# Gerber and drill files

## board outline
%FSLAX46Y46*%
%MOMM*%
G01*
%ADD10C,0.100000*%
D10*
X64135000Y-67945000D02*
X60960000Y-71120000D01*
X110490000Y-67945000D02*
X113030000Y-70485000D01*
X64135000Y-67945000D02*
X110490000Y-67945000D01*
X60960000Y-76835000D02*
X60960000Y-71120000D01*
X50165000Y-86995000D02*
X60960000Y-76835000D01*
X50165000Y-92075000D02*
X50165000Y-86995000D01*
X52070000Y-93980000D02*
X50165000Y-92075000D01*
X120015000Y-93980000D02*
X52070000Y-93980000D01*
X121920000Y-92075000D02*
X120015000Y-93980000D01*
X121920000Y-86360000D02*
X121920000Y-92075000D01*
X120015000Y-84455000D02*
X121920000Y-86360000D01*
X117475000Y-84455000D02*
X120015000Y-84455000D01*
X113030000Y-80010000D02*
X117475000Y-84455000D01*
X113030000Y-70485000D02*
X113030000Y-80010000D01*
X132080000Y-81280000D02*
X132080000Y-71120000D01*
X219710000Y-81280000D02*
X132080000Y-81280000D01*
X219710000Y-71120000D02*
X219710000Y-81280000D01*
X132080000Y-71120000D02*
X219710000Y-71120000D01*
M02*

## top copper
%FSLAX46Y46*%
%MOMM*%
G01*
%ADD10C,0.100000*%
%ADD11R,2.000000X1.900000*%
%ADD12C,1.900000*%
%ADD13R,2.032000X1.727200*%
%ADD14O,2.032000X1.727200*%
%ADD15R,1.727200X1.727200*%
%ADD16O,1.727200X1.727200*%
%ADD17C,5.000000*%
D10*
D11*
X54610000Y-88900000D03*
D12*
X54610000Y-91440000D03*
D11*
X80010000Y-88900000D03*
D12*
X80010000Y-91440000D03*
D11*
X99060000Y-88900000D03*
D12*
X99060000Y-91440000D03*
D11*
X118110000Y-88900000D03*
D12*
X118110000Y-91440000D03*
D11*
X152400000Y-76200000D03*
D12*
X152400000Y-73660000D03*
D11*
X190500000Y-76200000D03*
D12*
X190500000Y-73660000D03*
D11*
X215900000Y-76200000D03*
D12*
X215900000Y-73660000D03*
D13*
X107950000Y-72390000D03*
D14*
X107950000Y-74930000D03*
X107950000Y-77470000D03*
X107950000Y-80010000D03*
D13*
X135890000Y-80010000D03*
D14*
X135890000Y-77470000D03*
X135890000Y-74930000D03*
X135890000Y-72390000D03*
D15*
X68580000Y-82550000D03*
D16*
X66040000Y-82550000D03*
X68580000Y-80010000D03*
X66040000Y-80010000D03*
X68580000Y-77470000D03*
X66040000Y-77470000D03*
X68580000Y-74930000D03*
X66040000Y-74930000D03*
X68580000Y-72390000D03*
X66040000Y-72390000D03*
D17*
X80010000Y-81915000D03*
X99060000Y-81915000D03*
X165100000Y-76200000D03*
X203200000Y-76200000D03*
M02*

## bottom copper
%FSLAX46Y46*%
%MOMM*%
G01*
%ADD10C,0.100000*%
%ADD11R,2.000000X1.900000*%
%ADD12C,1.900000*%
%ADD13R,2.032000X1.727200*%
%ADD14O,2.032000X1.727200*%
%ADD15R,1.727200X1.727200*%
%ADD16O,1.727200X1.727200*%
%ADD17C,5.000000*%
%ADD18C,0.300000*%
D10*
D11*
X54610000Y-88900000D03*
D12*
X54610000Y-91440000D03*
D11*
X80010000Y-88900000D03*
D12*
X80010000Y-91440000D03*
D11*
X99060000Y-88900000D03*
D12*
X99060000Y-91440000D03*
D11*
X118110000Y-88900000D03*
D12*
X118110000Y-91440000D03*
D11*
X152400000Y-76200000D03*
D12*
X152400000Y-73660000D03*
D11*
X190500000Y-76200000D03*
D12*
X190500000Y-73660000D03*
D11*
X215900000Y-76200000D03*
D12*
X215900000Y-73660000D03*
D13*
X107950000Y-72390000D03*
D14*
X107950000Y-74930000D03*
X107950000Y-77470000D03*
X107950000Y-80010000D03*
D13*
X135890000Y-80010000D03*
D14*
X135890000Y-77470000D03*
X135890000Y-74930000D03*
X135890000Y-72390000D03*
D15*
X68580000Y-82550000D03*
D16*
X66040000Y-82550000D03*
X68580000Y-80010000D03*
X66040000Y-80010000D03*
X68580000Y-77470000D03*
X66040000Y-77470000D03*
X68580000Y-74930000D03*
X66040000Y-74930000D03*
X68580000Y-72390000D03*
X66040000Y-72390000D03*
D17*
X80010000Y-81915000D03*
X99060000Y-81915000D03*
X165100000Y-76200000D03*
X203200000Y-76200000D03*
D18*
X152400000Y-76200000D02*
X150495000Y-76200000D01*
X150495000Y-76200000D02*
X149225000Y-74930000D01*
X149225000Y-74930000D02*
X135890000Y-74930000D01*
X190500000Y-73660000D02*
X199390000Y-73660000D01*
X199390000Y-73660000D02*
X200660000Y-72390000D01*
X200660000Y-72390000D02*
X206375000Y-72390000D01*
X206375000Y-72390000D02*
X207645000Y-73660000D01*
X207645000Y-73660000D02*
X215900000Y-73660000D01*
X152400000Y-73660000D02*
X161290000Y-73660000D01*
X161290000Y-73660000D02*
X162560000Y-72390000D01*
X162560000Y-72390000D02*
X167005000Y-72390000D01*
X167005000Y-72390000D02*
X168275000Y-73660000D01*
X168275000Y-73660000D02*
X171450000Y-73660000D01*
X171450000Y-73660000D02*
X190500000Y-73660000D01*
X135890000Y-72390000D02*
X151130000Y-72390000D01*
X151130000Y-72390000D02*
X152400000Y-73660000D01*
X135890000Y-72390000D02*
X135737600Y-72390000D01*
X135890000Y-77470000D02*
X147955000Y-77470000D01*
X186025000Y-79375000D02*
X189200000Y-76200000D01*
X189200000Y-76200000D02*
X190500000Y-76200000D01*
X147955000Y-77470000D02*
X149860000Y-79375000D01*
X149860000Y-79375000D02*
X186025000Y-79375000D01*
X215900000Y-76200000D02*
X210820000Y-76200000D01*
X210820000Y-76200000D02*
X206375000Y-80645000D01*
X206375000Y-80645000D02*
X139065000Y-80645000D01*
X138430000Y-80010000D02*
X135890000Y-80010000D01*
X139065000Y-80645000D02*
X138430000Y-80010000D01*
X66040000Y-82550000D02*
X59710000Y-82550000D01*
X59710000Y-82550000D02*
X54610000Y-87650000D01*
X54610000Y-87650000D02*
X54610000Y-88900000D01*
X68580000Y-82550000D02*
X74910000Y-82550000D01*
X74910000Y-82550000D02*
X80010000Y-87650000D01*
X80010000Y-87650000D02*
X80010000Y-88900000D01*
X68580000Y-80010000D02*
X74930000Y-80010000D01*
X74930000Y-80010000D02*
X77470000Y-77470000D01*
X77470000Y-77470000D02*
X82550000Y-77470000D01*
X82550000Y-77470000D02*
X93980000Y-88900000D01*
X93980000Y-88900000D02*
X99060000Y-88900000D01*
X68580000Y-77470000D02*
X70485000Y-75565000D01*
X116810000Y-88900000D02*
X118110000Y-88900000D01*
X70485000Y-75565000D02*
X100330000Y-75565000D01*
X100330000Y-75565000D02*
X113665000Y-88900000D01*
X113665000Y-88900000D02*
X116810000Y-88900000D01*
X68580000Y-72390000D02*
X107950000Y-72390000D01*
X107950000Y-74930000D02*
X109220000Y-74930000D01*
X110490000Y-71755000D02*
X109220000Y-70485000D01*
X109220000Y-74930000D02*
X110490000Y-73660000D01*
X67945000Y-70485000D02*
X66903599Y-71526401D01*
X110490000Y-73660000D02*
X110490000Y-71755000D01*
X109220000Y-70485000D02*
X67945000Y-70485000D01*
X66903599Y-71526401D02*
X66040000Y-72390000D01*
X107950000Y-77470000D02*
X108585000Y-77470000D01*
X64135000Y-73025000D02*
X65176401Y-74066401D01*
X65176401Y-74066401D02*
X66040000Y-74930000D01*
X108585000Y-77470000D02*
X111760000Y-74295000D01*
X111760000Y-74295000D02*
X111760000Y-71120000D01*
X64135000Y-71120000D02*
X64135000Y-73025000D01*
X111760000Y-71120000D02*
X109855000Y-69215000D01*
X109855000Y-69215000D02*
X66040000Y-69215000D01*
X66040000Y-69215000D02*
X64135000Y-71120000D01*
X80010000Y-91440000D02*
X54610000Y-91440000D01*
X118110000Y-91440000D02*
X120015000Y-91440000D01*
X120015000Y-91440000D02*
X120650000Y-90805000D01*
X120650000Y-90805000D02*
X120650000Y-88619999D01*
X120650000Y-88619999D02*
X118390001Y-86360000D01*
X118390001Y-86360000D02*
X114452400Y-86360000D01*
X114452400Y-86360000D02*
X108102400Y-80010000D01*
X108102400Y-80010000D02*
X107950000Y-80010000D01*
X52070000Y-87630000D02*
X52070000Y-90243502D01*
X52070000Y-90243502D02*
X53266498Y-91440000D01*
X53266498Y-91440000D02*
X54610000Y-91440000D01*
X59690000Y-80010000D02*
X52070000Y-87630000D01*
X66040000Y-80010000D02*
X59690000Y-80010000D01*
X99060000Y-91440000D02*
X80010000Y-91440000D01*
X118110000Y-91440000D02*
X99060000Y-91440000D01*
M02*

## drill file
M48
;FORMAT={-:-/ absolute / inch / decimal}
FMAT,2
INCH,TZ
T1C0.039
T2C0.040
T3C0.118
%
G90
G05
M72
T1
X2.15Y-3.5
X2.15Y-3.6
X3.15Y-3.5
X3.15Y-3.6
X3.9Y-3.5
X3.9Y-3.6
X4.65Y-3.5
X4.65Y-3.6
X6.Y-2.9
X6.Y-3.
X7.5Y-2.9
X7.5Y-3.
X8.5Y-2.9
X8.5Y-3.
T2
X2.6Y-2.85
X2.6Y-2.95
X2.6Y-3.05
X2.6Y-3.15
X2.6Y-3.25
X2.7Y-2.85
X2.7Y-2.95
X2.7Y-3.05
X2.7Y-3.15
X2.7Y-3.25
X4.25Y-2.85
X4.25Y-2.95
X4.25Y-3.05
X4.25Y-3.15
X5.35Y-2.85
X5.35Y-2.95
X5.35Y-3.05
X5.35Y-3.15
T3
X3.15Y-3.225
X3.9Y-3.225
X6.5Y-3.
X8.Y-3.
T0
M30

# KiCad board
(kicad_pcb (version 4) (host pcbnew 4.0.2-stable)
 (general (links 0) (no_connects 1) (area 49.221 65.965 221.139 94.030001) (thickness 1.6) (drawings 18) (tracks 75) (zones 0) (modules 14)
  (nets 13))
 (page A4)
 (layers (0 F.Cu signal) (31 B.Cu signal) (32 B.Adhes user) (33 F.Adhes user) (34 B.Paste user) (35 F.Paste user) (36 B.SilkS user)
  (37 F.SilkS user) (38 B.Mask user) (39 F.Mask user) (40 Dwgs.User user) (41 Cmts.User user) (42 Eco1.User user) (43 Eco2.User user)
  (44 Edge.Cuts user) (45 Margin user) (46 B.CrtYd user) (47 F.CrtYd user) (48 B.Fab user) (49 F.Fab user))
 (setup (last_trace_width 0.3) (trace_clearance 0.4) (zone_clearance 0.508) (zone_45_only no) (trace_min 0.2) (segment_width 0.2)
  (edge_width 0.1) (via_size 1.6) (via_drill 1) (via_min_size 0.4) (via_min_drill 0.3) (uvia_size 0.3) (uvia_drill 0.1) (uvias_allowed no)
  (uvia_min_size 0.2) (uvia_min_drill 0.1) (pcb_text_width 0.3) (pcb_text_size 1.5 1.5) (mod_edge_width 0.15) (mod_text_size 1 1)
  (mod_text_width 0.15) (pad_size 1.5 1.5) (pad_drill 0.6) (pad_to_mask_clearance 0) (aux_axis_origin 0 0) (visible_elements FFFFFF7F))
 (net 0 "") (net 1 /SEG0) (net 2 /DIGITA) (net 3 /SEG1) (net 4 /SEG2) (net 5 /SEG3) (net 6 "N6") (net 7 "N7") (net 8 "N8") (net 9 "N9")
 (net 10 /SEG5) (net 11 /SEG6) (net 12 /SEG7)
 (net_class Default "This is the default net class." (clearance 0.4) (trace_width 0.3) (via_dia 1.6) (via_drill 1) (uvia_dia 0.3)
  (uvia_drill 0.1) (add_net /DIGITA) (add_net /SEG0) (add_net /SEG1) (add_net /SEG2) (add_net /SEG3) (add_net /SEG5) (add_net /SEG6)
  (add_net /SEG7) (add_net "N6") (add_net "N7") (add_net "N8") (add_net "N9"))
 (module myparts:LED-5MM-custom (layer F.Cu) (at 54.61 88.9 270)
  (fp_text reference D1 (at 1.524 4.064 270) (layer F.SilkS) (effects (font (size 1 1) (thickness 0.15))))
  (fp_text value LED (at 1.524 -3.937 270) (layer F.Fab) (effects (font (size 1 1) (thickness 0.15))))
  (pad 1 thru_hole rect (at 0 0) (size 2 1.9) (drill 1.00076) (layers *.Cu *.Mask F.SilkS) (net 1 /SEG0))
  (pad 2 thru_hole circle (at 2.54 0 270) (size 1.9 1.9) (drill 1.00076) (layers *.Cu *.Mask F.SilkS) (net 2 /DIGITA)))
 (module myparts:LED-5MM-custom (layer F.Cu) (at 80.01 88.9 270)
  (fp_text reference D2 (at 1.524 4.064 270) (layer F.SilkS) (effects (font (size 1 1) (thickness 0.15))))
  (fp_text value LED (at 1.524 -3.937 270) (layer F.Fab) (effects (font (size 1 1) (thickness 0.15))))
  (pad 1 thru_hole rect (at 0 0) (size 2 1.9) (drill 1.00076) (layers *.Cu *.Mask F.SilkS) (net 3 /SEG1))
  (pad 2 thru_hole circle (at 2.54 0 270) (size 1.9 1.9) (drill 1.00076) (layers *.Cu *.Mask F.SilkS) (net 2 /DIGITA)))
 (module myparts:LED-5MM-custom (layer F.Cu) (at 99.06 88.9 270)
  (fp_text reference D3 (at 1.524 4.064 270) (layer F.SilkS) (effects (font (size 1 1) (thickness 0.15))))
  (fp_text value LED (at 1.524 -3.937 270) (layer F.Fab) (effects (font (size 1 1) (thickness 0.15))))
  (pad 1 thru_hole rect (at 0 0) (size 2 1.9) (drill 1.00076) (layers *.Cu *.Mask F.SilkS) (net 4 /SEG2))
  (pad 2 thru_hole circle (at 2.54 0 270) (size 1.9 1.9) (drill 1.00076) (layers *.Cu *.Mask F.SilkS) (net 2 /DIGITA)))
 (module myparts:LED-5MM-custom (layer F.Cu) (at 118.11 88.9 270)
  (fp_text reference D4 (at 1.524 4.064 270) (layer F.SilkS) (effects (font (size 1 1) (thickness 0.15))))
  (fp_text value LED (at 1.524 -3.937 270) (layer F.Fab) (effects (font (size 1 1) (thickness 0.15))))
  (pad 1 thru_hole rect (at 0 0) (size 2 1.9) (drill 1.00076) (layers *.Cu *.Mask F.SilkS) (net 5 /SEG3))
  (pad 2 thru_hole circle (at 2.54 0 270) (size 1.9 1.9) (drill 1.00076) (layers *.Cu *.Mask F.SilkS) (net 2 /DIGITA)))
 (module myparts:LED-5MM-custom (layer F.Cu) (at 152.4 76.2 90)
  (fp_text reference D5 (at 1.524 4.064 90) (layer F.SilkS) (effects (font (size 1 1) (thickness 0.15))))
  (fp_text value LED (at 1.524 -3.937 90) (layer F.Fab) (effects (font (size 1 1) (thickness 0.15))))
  (pad 1 thru_hole rect (at 0 0 180) (size 2 1.9) (drill 1.00076) (layers *.Cu *.Mask F.SilkS) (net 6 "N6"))
  (pad 2 thru_hole circle (at 2.54 0 90) (size 1.9 1.9) (drill 1.00076) (layers *.Cu *.Mask F.SilkS) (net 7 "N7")))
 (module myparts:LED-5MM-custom (layer F.Cu) (at 190.5 76.2 90)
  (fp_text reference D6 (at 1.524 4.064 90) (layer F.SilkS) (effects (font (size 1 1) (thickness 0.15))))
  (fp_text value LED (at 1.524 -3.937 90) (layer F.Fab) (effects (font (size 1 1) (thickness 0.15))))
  (pad 1 thru_hole rect (at 0 0 180) (size 2 1.9) (drill 1.00076) (layers *.Cu *.Mask F.SilkS) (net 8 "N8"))
  (pad 2 thru_hole circle (at 2.54 0 90) (size 1.9 1.9) (drill 1.00076) (layers *.Cu *.Mask F.SilkS) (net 7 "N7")))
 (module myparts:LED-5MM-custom (layer F.Cu) (at 215.9 76.2 90)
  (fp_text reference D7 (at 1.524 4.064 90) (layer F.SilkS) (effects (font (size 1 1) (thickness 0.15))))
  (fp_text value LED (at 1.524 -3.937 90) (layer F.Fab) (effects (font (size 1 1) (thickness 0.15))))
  (pad 1 thru_hole rect (at 0 0 180) (size 2 1.9) (drill 1.00076) (layers *.Cu *.Mask F.SilkS) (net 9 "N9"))
  (pad 2 thru_hole circle (at 2.54 0 90) (size 1.9 1.9) (drill 1.00076) (layers *.Cu *.Mask F.SilkS) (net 7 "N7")))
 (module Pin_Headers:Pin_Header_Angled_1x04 (layer F.Cu) (at 107.95 72.39)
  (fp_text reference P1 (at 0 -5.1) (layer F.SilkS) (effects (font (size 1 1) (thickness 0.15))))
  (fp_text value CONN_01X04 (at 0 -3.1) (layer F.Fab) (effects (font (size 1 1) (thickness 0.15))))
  (pad 1 thru_hole rect (at 0 0) (size 2.032 1.7272) (drill 1.016) (layers *.Cu *.Mask F.SilkS) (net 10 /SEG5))
  (pad 2 thru_hole oval (at 0 2.54) (size 2.032 1.7272) (drill 1.016) (layers *.Cu *.Mask F.SilkS) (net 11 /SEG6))
  (pad 3 thru_hole oval (at 0 5.08) (size 2.032 1.7272) (drill 1.016) (layers *.Cu *.Mask F.SilkS) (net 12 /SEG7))
  (pad 4 thru_hole oval (at 0 7.62) (size 2.032 1.7272) (drill 1.016) (layers *.Cu *.Mask F.SilkS) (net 2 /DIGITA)))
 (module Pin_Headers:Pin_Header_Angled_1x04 (layer F.Cu) (at 135.89 80.01 180)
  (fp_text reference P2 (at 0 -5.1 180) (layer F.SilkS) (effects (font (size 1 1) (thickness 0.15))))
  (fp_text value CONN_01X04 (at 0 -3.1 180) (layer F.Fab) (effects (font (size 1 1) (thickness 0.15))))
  (pad 1 thru_hole rect (at 0 0 180) (size 2.032 1.7272) (drill 1.016) (layers *.Cu *.Mask F.SilkS) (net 9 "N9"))
  (pad 2 thru_hole oval (at 0 2.54 180) (size 2.032 1.7272) (drill 1.016) (layers *.Cu *.Mask F.SilkS) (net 8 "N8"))
  (pad 3 thru_hole oval (at 0 5.08 180) (size 2.032 1.7272) (drill 1.016) (layers *.Cu *.Mask F.SilkS) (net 6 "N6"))
  (pad 4 thru_hole oval (at 0 7.62 180) (size 2.032 1.7272) (drill 1.016) (layers *.Cu *.Mask F.SilkS) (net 7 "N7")))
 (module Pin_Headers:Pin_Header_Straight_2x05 (layer F.Cu) (at 68.58 82.55 180)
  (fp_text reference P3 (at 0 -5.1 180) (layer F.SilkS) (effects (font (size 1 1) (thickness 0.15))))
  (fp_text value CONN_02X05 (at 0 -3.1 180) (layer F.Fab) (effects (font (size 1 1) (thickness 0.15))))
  (pad 1 thru_hole rect (at 0 0 180) (size 1.7272 1.7272) (drill 1.016) (layers *.Cu *.Mask F.SilkS) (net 3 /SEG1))
  (pad 2 thru_hole oval (at 2.54 0 180) (size 1.7272 1.7272) (drill 1.016) (layers *.Cu *.Mask F.SilkS) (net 1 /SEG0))
  (pad 3 thru_hole oval (at 0 2.54 180) (size 1.7272 1.7272) (drill 1.016) (layers *.Cu *.Mask F.SilkS) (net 4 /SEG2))
  (pad 4 thru_hole oval (at 2.54 2.54 180) (size 1.7272 1.7272) (drill 1.016) (layers *.Cu *.Mask F.SilkS) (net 2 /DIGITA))
  (pad 5 thru_hole oval (at 0 5.08 180) (size 1.7272 1.7272) (drill 1.016) (layers *.Cu *.Mask F.SilkS) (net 5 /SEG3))
  (pad 6 thru_hole oval (at 2.54 5.08 180) (size 1.7272 1.7272) (drill 1.016) (layers *.Cu *.Mask F.SilkS))
  (pad 7 thru_hole oval (at 0 7.62 180) (size 1.7272 1.7272) (drill 1.016) (layers *.Cu *.Mask F.SilkS))
  (pad 8 thru_hole oval (at 2.54 7.62 180) (size 1.7272 1.7272) (drill 1.016) (layers *.Cu *.Mask F.SilkS) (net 12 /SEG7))
  (pad 9 thru_hole oval (at 0 10.16 180) (size 1.7272 1.7272) (drill 1.016) (layers *.Cu *.Mask F.SilkS) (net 10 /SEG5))
  (pad 10 thru_hole oval (at 2.54 10.16 180) (size 1.7272 1.7272) (drill 1.016) (layers *.Cu *.Mask F.SilkS) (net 11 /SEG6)))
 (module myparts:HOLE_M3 (layer F.Cu) (at 80.01 81.915)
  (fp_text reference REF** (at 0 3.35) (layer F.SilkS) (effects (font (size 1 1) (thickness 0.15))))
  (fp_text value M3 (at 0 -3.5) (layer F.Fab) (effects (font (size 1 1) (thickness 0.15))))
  (pad 1 thru_hole circle (at 0 0) (size 5 5) (drill 3) (layers *.Cu *.Mask F.SilkS)))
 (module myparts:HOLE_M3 (layer F.Cu) (at 99.06 81.915)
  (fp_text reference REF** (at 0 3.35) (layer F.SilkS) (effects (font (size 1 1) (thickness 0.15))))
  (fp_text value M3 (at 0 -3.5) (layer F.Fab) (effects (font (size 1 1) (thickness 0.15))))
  (pad 1 thru_hole circle (at 0 0) (size 5 5) (drill 3) (layers *.Cu *.Mask F.SilkS)))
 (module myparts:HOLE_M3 (layer F.Cu) (at 165.1 76.2)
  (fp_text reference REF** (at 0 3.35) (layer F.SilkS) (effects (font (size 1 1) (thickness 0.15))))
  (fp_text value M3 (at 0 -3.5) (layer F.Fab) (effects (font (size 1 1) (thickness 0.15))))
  (pad 1 thru_hole circle (at 0 0) (size 5 5) (drill 3) (layers *.Cu *.Mask F.SilkS)))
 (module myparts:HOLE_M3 (layer F.Cu) (at 203.2 76.2)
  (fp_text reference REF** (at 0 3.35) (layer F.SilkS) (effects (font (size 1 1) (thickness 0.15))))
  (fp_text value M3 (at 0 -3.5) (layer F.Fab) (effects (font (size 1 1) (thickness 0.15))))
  (pad 1 thru_hole circle (at 0 0) (size 5 5) (drill 3) (layers *.Cu *.Mask F.SilkS)))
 (gr_line (start 64.135 67.945) (end 60.96 71.12) (layer Edge.Cuts) (width 0.1))
 (gr_line (start 110.49 67.945) (end 113.03 70.485) (layer Edge.Cuts) (width 0.1))
 (gr_line (start 64.135 67.945) (end 110.49 67.945) (layer Edge.Cuts) (width 0.1))
 (gr_line (start 60.96 76.835) (end 60.96 71.12) (layer Edge.Cuts) (width 0.1))
 (gr_line (start 50.165 86.995) (end 60.96 76.835) (layer Edge.Cuts) (width 0.1))
 (gr_line (start 50.165 92.075) (end 50.165 86.995) (layer Edge.Cuts) (width 0.1))
 (gr_line (start 52.07 93.98) (end 50.165 92.075) (layer Edge.Cuts) (width 0.1))
 (gr_line (start 120.015 93.98) (end 52.07 93.98) (layer Edge.Cuts) (width 0.1))
 (gr_line (start 121.92 92.075) (end 120.015 93.98) (layer Edge.Cuts) (width 0.1))
 (gr_line (start 121.92 86.36) (end 121.92 92.075) (layer Edge.Cuts) (width 0.1))
 (gr_line (start 120.015 84.455) (end 121.92 86.36) (layer Edge.Cuts) (width 0.1))
 (gr_line (start 117.475 84.455) (end 120.015 84.455) (layer Edge.Cuts) (width 0.1))
 (gr_line (start 113.03 80.01) (end 117.475 84.455) (layer Edge.Cuts) (width 0.1))
 (gr_line (start 113.03 70.485) (end 113.03 80.01) (layer Edge.Cuts) (width 0.1))
 (gr_line (start 132.08 81.28) (end 132.08 71.12) (layer Edge.Cuts) (width 0.1))
 (gr_line (start 219.71 81.28) (end 132.08 81.28) (layer Edge.Cuts) (width 0.1))
 (gr_line (start 219.71 71.12) (end 219.71 81.28) (layer Edge.Cuts) (width 0.1))
 (gr_line (start 132.08 71.12) (end 219.71 71.12) (layer Edge.Cuts) (width 0.1))
 (segment (start 152.4 76.2) (end 150.495 76.2) (width 0.3) (layer B.Cu) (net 6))
 (segment (start 150.495 76.2) (end 149.225 74.93) (width 0.3) (layer B.Cu) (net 6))
 (segment (start 149.225 74.93) (end 135.89 74.93) (width 0.3) (layer B.Cu) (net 6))
 (segment (start 190.5 73.66) (end 199.39 73.66) (width 0.3) (layer B.Cu) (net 7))
 (segment (start 199.39 73.66) (end 200.66 72.39) (width 0.3) (layer B.Cu) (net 7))
 (segment (start 200.66 72.39) (end 206.375 72.39) (width 0.3) (layer B.Cu) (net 7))
 (segment (start 206.375 72.39) (end 207.645 73.66) (width 0.3) (layer B.Cu) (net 7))
 (segment (start 207.645 73.66) (end 215.9 73.66) (width 0.3) (layer B.Cu) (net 7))
 (segment (start 152.4 73.66) (end 161.29 73.66) (width 0.3) (layer B.Cu) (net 7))
 (segment (start 161.29 73.66) (end 162.56 72.39) (width 0.3) (layer B.Cu) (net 7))
 (segment (start 162.56 72.39) (end 167.005 72.39) (width 0.3) (layer B.Cu) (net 7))
 (segment (start 167.005 72.39) (end 168.275 73.66) (width 0.3) (layer B.Cu) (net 7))
 (segment (start 168.275 73.66) (end 171.45 73.66) (width 0.3) (layer B.Cu) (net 7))
 (segment (start 171.45 73.66) (end 190.5 73.66) (width 0.3) (layer B.Cu) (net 7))
 (segment (start 135.89 72.39) (end 151.13 72.39) (width 0.3) (layer B.Cu) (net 7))
 (segment (start 151.13 72.39) (end 152.4 73.66) (width 0.3) (layer B.Cu) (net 7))
 (segment (start 135.89 72.39) (end 135.7376 72.39) (width 0.3) (layer B.Cu) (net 7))
 (segment (start 135.89 77.47) (end 147.955 77.47) (width 0.3) (layer B.Cu) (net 8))
 (segment (start 186.025 79.375) (end 189.2 76.2) (width 0.3) (layer B.Cu) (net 8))
 (segment (start 189.2 76.2) (end 190.5 76.2) (width 0.3) (layer B.Cu) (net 8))
 (segment (start 147.955 77.47) (end 149.86 79.375) (width 0.3) (layer B.Cu) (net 8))
 (segment (start 149.86 79.375) (end 186.025 79.375) (width 0.3) (layer B.Cu) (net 8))
 (segment (start 215.9 76.2) (end 210.82 76.2) (width 0.3) (layer B.Cu) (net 9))
 (segment (start 210.82 76.2) (end 206.375 80.645) (width 0.3) (layer B.Cu) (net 9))
 (segment (start 206.375 80.645) (end 139.065 80.645) (width 0.3) (layer B.Cu) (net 9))
 (segment (start 138.43 80.01) (end 135.89 80.01) (width 0.3) (layer B.Cu) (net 9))
 (segment (start 139.065 80.645) (end 138.43 80.01) (width 0.3) (layer B.Cu) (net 9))
 (segment (start 66.04 82.55) (end 59.71 82.55) (width 0.3) (layer B.Cu) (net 1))
 (segment (start 59.71 82.55) (end 54.61 87.65) (width 0.3) (layer B.Cu) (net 1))
 (segment (start 54.61 87.65) (end 54.61 88.9) (width 0.3) (layer B.Cu) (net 1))
 (segment (start 68.58 82.55) (end 74.91 82.55) (width 0.3) (layer B.Cu) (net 3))
 (segment (start 74.91 82.55) (end 80.01 87.65) (width 0.3) (layer B.Cu) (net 3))
 (segment (start 80.01 87.65) (end 80.01 88.9) (width 0.3) (layer B.Cu) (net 3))
 (segment (start 68.58 80.01) (end 74.93 80.01) (width 0.3) (layer B.Cu) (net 4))
 (segment (start 74.93 80.01) (end 77.47 77.47) (width 0.3) (layer B.Cu) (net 4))
 (segment (start 77.47 77.47) (end 82.55 77.47) (width 0.3) (layer B.Cu) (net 4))
 (segment (start 82.55 77.47) (end 93.98 88.9) (width 0.3) (layer B.Cu) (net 4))
 (segment (start 93.98 88.9) (end 99.06 88.9) (width 0.3) (layer B.Cu) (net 4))
 (segment (start 68.58 77.47) (end 70.485 75.565) (width 0.3) (layer B.Cu) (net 5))
 (segment (start 116.81 88.9) (end 118.11 88.9) (width 0.3) (layer B.Cu) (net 5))
 (segment (start 70.485 75.565) (end 100.33 75.565) (width 0.3) (layer B.Cu) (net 5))
 (segment (start 100.33 75.565) (end 113.665 88.9) (width 0.3) (layer B.Cu) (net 5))
 (segment (start 113.665 88.9) (end 116.81 88.9) (width 0.3) (layer B.Cu) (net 5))
 (segment (start 68.58 72.39) (end 107.95 72.39) (width 0.3) (layer B.Cu) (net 10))
 (segment (start 107.95 74.93) (end 109.22 74.93) (width 0.3) (layer B.Cu) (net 11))
 (segment (start 110.49 71.755) (end 109.22 70.485) (width 0.3) (layer B.Cu) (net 11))
 (segment (start 109.22 74.93) (end 110.49 73.66) (width 0.3) (layer B.Cu) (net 11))
 (segment (start 67.945 70.485) (end 66.903599 71.526401) (width 0.3) (layer B.Cu) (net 11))
 (segment (start 110.49 73.66) (end 110.49 71.755) (width 0.3) (layer B.Cu) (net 11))
 (segment (start 109.22 70.485) (end 67.945 70.485) (width 0.3) (layer B.Cu) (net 11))
 (segment (start 66.903599 71.526401) (end 66.04 72.39) (width 0.3) (layer B.Cu) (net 11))
 (segment (start 107.95 77.47) (end 108.585 77.47) (width 0.3) (layer B.Cu) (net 12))
 (segment (start 64.135 73.025) (end 65.176401 74.066401) (width 0.3) (layer B.Cu) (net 12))
 (segment (start 65.176401 74.066401) (end 66.04 74.93) (width 0.3) (layer B.Cu) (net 12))
 (segment (start 108.585 77.47) (end 111.76 74.295) (width 0.3) (layer B.Cu) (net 12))
 (segment (start 111.76 74.295) (end 111.76 71.12) (width 0.3) (layer B.Cu) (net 12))
 (segment (start 64.135 71.12) (end 64.135 73.025) (width 0.3) (layer B.Cu) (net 12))
 (segment (start 111.76 71.12) (end 109.855 69.215) (width 0.3) (layer B.Cu) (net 12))
 (segment (start 109.855 69.215) (end 66.04 69.215) (width 0.3) (layer B.Cu) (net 12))
 (segment (start 66.04 69.215) (end 64.135 71.12) (width 0.3) (layer B.Cu) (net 12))
 (segment (start 80.01 91.44) (end 54.61 91.44) (width 0.3) (layer B.Cu) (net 2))
 (segment (start 118.11 91.44) (end 120.015 91.44) (width 0.3) (layer B.Cu) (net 2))
 (segment (start 120.015 91.44) (end 120.65 90.805) (width 0.3) (layer B.Cu) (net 2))
 (segment (start 120.65 90.805) (end 120.65 88.619999) (width 0.3) (layer B.Cu) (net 2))
 (segment (start 120.65 88.619999) (end 118.390001 86.36) (width 0.3) (layer B.Cu) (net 2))
 (segment (start 118.390001 86.36) (end 114.4524 86.36) (width 0.3) (layer B.Cu) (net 2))
 (segment (start 114.4524 86.36) (end 108.1024 80.01) (width 0.3) (layer B.Cu) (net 2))
 (segment (start 108.1024 80.01) (end 107.95 80.01) (width 0.3) (layer B.Cu) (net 2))
 (segment (start 52.07 87.63) (end 52.07 90.243502) (width 0.3) (layer B.Cu) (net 2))
 (segment (start 52.07 90.243502) (end 53.266498 91.44) (width 0.3) (layer B.Cu) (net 2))
 (segment (start 53.266498 91.44) (end 54.61 91.44) (width 0.3) (layer B.Cu) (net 2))
 (segment (start 59.69 80.01) (end 52.07 87.63) (width 0.3) (layer B.Cu) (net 2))
 (segment (start 66.04 80.01) (end 59.69 80.01) (width 0.3) (layer B.Cu) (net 2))
 (segment (start 99.06 91.44) (end 80.01 91.44) (width 0.3) (layer B.Cu) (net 2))
 (segment (start 118.11 91.44) (end 99.06 91.44) (width 0.3) (layer B.Cu) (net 2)))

